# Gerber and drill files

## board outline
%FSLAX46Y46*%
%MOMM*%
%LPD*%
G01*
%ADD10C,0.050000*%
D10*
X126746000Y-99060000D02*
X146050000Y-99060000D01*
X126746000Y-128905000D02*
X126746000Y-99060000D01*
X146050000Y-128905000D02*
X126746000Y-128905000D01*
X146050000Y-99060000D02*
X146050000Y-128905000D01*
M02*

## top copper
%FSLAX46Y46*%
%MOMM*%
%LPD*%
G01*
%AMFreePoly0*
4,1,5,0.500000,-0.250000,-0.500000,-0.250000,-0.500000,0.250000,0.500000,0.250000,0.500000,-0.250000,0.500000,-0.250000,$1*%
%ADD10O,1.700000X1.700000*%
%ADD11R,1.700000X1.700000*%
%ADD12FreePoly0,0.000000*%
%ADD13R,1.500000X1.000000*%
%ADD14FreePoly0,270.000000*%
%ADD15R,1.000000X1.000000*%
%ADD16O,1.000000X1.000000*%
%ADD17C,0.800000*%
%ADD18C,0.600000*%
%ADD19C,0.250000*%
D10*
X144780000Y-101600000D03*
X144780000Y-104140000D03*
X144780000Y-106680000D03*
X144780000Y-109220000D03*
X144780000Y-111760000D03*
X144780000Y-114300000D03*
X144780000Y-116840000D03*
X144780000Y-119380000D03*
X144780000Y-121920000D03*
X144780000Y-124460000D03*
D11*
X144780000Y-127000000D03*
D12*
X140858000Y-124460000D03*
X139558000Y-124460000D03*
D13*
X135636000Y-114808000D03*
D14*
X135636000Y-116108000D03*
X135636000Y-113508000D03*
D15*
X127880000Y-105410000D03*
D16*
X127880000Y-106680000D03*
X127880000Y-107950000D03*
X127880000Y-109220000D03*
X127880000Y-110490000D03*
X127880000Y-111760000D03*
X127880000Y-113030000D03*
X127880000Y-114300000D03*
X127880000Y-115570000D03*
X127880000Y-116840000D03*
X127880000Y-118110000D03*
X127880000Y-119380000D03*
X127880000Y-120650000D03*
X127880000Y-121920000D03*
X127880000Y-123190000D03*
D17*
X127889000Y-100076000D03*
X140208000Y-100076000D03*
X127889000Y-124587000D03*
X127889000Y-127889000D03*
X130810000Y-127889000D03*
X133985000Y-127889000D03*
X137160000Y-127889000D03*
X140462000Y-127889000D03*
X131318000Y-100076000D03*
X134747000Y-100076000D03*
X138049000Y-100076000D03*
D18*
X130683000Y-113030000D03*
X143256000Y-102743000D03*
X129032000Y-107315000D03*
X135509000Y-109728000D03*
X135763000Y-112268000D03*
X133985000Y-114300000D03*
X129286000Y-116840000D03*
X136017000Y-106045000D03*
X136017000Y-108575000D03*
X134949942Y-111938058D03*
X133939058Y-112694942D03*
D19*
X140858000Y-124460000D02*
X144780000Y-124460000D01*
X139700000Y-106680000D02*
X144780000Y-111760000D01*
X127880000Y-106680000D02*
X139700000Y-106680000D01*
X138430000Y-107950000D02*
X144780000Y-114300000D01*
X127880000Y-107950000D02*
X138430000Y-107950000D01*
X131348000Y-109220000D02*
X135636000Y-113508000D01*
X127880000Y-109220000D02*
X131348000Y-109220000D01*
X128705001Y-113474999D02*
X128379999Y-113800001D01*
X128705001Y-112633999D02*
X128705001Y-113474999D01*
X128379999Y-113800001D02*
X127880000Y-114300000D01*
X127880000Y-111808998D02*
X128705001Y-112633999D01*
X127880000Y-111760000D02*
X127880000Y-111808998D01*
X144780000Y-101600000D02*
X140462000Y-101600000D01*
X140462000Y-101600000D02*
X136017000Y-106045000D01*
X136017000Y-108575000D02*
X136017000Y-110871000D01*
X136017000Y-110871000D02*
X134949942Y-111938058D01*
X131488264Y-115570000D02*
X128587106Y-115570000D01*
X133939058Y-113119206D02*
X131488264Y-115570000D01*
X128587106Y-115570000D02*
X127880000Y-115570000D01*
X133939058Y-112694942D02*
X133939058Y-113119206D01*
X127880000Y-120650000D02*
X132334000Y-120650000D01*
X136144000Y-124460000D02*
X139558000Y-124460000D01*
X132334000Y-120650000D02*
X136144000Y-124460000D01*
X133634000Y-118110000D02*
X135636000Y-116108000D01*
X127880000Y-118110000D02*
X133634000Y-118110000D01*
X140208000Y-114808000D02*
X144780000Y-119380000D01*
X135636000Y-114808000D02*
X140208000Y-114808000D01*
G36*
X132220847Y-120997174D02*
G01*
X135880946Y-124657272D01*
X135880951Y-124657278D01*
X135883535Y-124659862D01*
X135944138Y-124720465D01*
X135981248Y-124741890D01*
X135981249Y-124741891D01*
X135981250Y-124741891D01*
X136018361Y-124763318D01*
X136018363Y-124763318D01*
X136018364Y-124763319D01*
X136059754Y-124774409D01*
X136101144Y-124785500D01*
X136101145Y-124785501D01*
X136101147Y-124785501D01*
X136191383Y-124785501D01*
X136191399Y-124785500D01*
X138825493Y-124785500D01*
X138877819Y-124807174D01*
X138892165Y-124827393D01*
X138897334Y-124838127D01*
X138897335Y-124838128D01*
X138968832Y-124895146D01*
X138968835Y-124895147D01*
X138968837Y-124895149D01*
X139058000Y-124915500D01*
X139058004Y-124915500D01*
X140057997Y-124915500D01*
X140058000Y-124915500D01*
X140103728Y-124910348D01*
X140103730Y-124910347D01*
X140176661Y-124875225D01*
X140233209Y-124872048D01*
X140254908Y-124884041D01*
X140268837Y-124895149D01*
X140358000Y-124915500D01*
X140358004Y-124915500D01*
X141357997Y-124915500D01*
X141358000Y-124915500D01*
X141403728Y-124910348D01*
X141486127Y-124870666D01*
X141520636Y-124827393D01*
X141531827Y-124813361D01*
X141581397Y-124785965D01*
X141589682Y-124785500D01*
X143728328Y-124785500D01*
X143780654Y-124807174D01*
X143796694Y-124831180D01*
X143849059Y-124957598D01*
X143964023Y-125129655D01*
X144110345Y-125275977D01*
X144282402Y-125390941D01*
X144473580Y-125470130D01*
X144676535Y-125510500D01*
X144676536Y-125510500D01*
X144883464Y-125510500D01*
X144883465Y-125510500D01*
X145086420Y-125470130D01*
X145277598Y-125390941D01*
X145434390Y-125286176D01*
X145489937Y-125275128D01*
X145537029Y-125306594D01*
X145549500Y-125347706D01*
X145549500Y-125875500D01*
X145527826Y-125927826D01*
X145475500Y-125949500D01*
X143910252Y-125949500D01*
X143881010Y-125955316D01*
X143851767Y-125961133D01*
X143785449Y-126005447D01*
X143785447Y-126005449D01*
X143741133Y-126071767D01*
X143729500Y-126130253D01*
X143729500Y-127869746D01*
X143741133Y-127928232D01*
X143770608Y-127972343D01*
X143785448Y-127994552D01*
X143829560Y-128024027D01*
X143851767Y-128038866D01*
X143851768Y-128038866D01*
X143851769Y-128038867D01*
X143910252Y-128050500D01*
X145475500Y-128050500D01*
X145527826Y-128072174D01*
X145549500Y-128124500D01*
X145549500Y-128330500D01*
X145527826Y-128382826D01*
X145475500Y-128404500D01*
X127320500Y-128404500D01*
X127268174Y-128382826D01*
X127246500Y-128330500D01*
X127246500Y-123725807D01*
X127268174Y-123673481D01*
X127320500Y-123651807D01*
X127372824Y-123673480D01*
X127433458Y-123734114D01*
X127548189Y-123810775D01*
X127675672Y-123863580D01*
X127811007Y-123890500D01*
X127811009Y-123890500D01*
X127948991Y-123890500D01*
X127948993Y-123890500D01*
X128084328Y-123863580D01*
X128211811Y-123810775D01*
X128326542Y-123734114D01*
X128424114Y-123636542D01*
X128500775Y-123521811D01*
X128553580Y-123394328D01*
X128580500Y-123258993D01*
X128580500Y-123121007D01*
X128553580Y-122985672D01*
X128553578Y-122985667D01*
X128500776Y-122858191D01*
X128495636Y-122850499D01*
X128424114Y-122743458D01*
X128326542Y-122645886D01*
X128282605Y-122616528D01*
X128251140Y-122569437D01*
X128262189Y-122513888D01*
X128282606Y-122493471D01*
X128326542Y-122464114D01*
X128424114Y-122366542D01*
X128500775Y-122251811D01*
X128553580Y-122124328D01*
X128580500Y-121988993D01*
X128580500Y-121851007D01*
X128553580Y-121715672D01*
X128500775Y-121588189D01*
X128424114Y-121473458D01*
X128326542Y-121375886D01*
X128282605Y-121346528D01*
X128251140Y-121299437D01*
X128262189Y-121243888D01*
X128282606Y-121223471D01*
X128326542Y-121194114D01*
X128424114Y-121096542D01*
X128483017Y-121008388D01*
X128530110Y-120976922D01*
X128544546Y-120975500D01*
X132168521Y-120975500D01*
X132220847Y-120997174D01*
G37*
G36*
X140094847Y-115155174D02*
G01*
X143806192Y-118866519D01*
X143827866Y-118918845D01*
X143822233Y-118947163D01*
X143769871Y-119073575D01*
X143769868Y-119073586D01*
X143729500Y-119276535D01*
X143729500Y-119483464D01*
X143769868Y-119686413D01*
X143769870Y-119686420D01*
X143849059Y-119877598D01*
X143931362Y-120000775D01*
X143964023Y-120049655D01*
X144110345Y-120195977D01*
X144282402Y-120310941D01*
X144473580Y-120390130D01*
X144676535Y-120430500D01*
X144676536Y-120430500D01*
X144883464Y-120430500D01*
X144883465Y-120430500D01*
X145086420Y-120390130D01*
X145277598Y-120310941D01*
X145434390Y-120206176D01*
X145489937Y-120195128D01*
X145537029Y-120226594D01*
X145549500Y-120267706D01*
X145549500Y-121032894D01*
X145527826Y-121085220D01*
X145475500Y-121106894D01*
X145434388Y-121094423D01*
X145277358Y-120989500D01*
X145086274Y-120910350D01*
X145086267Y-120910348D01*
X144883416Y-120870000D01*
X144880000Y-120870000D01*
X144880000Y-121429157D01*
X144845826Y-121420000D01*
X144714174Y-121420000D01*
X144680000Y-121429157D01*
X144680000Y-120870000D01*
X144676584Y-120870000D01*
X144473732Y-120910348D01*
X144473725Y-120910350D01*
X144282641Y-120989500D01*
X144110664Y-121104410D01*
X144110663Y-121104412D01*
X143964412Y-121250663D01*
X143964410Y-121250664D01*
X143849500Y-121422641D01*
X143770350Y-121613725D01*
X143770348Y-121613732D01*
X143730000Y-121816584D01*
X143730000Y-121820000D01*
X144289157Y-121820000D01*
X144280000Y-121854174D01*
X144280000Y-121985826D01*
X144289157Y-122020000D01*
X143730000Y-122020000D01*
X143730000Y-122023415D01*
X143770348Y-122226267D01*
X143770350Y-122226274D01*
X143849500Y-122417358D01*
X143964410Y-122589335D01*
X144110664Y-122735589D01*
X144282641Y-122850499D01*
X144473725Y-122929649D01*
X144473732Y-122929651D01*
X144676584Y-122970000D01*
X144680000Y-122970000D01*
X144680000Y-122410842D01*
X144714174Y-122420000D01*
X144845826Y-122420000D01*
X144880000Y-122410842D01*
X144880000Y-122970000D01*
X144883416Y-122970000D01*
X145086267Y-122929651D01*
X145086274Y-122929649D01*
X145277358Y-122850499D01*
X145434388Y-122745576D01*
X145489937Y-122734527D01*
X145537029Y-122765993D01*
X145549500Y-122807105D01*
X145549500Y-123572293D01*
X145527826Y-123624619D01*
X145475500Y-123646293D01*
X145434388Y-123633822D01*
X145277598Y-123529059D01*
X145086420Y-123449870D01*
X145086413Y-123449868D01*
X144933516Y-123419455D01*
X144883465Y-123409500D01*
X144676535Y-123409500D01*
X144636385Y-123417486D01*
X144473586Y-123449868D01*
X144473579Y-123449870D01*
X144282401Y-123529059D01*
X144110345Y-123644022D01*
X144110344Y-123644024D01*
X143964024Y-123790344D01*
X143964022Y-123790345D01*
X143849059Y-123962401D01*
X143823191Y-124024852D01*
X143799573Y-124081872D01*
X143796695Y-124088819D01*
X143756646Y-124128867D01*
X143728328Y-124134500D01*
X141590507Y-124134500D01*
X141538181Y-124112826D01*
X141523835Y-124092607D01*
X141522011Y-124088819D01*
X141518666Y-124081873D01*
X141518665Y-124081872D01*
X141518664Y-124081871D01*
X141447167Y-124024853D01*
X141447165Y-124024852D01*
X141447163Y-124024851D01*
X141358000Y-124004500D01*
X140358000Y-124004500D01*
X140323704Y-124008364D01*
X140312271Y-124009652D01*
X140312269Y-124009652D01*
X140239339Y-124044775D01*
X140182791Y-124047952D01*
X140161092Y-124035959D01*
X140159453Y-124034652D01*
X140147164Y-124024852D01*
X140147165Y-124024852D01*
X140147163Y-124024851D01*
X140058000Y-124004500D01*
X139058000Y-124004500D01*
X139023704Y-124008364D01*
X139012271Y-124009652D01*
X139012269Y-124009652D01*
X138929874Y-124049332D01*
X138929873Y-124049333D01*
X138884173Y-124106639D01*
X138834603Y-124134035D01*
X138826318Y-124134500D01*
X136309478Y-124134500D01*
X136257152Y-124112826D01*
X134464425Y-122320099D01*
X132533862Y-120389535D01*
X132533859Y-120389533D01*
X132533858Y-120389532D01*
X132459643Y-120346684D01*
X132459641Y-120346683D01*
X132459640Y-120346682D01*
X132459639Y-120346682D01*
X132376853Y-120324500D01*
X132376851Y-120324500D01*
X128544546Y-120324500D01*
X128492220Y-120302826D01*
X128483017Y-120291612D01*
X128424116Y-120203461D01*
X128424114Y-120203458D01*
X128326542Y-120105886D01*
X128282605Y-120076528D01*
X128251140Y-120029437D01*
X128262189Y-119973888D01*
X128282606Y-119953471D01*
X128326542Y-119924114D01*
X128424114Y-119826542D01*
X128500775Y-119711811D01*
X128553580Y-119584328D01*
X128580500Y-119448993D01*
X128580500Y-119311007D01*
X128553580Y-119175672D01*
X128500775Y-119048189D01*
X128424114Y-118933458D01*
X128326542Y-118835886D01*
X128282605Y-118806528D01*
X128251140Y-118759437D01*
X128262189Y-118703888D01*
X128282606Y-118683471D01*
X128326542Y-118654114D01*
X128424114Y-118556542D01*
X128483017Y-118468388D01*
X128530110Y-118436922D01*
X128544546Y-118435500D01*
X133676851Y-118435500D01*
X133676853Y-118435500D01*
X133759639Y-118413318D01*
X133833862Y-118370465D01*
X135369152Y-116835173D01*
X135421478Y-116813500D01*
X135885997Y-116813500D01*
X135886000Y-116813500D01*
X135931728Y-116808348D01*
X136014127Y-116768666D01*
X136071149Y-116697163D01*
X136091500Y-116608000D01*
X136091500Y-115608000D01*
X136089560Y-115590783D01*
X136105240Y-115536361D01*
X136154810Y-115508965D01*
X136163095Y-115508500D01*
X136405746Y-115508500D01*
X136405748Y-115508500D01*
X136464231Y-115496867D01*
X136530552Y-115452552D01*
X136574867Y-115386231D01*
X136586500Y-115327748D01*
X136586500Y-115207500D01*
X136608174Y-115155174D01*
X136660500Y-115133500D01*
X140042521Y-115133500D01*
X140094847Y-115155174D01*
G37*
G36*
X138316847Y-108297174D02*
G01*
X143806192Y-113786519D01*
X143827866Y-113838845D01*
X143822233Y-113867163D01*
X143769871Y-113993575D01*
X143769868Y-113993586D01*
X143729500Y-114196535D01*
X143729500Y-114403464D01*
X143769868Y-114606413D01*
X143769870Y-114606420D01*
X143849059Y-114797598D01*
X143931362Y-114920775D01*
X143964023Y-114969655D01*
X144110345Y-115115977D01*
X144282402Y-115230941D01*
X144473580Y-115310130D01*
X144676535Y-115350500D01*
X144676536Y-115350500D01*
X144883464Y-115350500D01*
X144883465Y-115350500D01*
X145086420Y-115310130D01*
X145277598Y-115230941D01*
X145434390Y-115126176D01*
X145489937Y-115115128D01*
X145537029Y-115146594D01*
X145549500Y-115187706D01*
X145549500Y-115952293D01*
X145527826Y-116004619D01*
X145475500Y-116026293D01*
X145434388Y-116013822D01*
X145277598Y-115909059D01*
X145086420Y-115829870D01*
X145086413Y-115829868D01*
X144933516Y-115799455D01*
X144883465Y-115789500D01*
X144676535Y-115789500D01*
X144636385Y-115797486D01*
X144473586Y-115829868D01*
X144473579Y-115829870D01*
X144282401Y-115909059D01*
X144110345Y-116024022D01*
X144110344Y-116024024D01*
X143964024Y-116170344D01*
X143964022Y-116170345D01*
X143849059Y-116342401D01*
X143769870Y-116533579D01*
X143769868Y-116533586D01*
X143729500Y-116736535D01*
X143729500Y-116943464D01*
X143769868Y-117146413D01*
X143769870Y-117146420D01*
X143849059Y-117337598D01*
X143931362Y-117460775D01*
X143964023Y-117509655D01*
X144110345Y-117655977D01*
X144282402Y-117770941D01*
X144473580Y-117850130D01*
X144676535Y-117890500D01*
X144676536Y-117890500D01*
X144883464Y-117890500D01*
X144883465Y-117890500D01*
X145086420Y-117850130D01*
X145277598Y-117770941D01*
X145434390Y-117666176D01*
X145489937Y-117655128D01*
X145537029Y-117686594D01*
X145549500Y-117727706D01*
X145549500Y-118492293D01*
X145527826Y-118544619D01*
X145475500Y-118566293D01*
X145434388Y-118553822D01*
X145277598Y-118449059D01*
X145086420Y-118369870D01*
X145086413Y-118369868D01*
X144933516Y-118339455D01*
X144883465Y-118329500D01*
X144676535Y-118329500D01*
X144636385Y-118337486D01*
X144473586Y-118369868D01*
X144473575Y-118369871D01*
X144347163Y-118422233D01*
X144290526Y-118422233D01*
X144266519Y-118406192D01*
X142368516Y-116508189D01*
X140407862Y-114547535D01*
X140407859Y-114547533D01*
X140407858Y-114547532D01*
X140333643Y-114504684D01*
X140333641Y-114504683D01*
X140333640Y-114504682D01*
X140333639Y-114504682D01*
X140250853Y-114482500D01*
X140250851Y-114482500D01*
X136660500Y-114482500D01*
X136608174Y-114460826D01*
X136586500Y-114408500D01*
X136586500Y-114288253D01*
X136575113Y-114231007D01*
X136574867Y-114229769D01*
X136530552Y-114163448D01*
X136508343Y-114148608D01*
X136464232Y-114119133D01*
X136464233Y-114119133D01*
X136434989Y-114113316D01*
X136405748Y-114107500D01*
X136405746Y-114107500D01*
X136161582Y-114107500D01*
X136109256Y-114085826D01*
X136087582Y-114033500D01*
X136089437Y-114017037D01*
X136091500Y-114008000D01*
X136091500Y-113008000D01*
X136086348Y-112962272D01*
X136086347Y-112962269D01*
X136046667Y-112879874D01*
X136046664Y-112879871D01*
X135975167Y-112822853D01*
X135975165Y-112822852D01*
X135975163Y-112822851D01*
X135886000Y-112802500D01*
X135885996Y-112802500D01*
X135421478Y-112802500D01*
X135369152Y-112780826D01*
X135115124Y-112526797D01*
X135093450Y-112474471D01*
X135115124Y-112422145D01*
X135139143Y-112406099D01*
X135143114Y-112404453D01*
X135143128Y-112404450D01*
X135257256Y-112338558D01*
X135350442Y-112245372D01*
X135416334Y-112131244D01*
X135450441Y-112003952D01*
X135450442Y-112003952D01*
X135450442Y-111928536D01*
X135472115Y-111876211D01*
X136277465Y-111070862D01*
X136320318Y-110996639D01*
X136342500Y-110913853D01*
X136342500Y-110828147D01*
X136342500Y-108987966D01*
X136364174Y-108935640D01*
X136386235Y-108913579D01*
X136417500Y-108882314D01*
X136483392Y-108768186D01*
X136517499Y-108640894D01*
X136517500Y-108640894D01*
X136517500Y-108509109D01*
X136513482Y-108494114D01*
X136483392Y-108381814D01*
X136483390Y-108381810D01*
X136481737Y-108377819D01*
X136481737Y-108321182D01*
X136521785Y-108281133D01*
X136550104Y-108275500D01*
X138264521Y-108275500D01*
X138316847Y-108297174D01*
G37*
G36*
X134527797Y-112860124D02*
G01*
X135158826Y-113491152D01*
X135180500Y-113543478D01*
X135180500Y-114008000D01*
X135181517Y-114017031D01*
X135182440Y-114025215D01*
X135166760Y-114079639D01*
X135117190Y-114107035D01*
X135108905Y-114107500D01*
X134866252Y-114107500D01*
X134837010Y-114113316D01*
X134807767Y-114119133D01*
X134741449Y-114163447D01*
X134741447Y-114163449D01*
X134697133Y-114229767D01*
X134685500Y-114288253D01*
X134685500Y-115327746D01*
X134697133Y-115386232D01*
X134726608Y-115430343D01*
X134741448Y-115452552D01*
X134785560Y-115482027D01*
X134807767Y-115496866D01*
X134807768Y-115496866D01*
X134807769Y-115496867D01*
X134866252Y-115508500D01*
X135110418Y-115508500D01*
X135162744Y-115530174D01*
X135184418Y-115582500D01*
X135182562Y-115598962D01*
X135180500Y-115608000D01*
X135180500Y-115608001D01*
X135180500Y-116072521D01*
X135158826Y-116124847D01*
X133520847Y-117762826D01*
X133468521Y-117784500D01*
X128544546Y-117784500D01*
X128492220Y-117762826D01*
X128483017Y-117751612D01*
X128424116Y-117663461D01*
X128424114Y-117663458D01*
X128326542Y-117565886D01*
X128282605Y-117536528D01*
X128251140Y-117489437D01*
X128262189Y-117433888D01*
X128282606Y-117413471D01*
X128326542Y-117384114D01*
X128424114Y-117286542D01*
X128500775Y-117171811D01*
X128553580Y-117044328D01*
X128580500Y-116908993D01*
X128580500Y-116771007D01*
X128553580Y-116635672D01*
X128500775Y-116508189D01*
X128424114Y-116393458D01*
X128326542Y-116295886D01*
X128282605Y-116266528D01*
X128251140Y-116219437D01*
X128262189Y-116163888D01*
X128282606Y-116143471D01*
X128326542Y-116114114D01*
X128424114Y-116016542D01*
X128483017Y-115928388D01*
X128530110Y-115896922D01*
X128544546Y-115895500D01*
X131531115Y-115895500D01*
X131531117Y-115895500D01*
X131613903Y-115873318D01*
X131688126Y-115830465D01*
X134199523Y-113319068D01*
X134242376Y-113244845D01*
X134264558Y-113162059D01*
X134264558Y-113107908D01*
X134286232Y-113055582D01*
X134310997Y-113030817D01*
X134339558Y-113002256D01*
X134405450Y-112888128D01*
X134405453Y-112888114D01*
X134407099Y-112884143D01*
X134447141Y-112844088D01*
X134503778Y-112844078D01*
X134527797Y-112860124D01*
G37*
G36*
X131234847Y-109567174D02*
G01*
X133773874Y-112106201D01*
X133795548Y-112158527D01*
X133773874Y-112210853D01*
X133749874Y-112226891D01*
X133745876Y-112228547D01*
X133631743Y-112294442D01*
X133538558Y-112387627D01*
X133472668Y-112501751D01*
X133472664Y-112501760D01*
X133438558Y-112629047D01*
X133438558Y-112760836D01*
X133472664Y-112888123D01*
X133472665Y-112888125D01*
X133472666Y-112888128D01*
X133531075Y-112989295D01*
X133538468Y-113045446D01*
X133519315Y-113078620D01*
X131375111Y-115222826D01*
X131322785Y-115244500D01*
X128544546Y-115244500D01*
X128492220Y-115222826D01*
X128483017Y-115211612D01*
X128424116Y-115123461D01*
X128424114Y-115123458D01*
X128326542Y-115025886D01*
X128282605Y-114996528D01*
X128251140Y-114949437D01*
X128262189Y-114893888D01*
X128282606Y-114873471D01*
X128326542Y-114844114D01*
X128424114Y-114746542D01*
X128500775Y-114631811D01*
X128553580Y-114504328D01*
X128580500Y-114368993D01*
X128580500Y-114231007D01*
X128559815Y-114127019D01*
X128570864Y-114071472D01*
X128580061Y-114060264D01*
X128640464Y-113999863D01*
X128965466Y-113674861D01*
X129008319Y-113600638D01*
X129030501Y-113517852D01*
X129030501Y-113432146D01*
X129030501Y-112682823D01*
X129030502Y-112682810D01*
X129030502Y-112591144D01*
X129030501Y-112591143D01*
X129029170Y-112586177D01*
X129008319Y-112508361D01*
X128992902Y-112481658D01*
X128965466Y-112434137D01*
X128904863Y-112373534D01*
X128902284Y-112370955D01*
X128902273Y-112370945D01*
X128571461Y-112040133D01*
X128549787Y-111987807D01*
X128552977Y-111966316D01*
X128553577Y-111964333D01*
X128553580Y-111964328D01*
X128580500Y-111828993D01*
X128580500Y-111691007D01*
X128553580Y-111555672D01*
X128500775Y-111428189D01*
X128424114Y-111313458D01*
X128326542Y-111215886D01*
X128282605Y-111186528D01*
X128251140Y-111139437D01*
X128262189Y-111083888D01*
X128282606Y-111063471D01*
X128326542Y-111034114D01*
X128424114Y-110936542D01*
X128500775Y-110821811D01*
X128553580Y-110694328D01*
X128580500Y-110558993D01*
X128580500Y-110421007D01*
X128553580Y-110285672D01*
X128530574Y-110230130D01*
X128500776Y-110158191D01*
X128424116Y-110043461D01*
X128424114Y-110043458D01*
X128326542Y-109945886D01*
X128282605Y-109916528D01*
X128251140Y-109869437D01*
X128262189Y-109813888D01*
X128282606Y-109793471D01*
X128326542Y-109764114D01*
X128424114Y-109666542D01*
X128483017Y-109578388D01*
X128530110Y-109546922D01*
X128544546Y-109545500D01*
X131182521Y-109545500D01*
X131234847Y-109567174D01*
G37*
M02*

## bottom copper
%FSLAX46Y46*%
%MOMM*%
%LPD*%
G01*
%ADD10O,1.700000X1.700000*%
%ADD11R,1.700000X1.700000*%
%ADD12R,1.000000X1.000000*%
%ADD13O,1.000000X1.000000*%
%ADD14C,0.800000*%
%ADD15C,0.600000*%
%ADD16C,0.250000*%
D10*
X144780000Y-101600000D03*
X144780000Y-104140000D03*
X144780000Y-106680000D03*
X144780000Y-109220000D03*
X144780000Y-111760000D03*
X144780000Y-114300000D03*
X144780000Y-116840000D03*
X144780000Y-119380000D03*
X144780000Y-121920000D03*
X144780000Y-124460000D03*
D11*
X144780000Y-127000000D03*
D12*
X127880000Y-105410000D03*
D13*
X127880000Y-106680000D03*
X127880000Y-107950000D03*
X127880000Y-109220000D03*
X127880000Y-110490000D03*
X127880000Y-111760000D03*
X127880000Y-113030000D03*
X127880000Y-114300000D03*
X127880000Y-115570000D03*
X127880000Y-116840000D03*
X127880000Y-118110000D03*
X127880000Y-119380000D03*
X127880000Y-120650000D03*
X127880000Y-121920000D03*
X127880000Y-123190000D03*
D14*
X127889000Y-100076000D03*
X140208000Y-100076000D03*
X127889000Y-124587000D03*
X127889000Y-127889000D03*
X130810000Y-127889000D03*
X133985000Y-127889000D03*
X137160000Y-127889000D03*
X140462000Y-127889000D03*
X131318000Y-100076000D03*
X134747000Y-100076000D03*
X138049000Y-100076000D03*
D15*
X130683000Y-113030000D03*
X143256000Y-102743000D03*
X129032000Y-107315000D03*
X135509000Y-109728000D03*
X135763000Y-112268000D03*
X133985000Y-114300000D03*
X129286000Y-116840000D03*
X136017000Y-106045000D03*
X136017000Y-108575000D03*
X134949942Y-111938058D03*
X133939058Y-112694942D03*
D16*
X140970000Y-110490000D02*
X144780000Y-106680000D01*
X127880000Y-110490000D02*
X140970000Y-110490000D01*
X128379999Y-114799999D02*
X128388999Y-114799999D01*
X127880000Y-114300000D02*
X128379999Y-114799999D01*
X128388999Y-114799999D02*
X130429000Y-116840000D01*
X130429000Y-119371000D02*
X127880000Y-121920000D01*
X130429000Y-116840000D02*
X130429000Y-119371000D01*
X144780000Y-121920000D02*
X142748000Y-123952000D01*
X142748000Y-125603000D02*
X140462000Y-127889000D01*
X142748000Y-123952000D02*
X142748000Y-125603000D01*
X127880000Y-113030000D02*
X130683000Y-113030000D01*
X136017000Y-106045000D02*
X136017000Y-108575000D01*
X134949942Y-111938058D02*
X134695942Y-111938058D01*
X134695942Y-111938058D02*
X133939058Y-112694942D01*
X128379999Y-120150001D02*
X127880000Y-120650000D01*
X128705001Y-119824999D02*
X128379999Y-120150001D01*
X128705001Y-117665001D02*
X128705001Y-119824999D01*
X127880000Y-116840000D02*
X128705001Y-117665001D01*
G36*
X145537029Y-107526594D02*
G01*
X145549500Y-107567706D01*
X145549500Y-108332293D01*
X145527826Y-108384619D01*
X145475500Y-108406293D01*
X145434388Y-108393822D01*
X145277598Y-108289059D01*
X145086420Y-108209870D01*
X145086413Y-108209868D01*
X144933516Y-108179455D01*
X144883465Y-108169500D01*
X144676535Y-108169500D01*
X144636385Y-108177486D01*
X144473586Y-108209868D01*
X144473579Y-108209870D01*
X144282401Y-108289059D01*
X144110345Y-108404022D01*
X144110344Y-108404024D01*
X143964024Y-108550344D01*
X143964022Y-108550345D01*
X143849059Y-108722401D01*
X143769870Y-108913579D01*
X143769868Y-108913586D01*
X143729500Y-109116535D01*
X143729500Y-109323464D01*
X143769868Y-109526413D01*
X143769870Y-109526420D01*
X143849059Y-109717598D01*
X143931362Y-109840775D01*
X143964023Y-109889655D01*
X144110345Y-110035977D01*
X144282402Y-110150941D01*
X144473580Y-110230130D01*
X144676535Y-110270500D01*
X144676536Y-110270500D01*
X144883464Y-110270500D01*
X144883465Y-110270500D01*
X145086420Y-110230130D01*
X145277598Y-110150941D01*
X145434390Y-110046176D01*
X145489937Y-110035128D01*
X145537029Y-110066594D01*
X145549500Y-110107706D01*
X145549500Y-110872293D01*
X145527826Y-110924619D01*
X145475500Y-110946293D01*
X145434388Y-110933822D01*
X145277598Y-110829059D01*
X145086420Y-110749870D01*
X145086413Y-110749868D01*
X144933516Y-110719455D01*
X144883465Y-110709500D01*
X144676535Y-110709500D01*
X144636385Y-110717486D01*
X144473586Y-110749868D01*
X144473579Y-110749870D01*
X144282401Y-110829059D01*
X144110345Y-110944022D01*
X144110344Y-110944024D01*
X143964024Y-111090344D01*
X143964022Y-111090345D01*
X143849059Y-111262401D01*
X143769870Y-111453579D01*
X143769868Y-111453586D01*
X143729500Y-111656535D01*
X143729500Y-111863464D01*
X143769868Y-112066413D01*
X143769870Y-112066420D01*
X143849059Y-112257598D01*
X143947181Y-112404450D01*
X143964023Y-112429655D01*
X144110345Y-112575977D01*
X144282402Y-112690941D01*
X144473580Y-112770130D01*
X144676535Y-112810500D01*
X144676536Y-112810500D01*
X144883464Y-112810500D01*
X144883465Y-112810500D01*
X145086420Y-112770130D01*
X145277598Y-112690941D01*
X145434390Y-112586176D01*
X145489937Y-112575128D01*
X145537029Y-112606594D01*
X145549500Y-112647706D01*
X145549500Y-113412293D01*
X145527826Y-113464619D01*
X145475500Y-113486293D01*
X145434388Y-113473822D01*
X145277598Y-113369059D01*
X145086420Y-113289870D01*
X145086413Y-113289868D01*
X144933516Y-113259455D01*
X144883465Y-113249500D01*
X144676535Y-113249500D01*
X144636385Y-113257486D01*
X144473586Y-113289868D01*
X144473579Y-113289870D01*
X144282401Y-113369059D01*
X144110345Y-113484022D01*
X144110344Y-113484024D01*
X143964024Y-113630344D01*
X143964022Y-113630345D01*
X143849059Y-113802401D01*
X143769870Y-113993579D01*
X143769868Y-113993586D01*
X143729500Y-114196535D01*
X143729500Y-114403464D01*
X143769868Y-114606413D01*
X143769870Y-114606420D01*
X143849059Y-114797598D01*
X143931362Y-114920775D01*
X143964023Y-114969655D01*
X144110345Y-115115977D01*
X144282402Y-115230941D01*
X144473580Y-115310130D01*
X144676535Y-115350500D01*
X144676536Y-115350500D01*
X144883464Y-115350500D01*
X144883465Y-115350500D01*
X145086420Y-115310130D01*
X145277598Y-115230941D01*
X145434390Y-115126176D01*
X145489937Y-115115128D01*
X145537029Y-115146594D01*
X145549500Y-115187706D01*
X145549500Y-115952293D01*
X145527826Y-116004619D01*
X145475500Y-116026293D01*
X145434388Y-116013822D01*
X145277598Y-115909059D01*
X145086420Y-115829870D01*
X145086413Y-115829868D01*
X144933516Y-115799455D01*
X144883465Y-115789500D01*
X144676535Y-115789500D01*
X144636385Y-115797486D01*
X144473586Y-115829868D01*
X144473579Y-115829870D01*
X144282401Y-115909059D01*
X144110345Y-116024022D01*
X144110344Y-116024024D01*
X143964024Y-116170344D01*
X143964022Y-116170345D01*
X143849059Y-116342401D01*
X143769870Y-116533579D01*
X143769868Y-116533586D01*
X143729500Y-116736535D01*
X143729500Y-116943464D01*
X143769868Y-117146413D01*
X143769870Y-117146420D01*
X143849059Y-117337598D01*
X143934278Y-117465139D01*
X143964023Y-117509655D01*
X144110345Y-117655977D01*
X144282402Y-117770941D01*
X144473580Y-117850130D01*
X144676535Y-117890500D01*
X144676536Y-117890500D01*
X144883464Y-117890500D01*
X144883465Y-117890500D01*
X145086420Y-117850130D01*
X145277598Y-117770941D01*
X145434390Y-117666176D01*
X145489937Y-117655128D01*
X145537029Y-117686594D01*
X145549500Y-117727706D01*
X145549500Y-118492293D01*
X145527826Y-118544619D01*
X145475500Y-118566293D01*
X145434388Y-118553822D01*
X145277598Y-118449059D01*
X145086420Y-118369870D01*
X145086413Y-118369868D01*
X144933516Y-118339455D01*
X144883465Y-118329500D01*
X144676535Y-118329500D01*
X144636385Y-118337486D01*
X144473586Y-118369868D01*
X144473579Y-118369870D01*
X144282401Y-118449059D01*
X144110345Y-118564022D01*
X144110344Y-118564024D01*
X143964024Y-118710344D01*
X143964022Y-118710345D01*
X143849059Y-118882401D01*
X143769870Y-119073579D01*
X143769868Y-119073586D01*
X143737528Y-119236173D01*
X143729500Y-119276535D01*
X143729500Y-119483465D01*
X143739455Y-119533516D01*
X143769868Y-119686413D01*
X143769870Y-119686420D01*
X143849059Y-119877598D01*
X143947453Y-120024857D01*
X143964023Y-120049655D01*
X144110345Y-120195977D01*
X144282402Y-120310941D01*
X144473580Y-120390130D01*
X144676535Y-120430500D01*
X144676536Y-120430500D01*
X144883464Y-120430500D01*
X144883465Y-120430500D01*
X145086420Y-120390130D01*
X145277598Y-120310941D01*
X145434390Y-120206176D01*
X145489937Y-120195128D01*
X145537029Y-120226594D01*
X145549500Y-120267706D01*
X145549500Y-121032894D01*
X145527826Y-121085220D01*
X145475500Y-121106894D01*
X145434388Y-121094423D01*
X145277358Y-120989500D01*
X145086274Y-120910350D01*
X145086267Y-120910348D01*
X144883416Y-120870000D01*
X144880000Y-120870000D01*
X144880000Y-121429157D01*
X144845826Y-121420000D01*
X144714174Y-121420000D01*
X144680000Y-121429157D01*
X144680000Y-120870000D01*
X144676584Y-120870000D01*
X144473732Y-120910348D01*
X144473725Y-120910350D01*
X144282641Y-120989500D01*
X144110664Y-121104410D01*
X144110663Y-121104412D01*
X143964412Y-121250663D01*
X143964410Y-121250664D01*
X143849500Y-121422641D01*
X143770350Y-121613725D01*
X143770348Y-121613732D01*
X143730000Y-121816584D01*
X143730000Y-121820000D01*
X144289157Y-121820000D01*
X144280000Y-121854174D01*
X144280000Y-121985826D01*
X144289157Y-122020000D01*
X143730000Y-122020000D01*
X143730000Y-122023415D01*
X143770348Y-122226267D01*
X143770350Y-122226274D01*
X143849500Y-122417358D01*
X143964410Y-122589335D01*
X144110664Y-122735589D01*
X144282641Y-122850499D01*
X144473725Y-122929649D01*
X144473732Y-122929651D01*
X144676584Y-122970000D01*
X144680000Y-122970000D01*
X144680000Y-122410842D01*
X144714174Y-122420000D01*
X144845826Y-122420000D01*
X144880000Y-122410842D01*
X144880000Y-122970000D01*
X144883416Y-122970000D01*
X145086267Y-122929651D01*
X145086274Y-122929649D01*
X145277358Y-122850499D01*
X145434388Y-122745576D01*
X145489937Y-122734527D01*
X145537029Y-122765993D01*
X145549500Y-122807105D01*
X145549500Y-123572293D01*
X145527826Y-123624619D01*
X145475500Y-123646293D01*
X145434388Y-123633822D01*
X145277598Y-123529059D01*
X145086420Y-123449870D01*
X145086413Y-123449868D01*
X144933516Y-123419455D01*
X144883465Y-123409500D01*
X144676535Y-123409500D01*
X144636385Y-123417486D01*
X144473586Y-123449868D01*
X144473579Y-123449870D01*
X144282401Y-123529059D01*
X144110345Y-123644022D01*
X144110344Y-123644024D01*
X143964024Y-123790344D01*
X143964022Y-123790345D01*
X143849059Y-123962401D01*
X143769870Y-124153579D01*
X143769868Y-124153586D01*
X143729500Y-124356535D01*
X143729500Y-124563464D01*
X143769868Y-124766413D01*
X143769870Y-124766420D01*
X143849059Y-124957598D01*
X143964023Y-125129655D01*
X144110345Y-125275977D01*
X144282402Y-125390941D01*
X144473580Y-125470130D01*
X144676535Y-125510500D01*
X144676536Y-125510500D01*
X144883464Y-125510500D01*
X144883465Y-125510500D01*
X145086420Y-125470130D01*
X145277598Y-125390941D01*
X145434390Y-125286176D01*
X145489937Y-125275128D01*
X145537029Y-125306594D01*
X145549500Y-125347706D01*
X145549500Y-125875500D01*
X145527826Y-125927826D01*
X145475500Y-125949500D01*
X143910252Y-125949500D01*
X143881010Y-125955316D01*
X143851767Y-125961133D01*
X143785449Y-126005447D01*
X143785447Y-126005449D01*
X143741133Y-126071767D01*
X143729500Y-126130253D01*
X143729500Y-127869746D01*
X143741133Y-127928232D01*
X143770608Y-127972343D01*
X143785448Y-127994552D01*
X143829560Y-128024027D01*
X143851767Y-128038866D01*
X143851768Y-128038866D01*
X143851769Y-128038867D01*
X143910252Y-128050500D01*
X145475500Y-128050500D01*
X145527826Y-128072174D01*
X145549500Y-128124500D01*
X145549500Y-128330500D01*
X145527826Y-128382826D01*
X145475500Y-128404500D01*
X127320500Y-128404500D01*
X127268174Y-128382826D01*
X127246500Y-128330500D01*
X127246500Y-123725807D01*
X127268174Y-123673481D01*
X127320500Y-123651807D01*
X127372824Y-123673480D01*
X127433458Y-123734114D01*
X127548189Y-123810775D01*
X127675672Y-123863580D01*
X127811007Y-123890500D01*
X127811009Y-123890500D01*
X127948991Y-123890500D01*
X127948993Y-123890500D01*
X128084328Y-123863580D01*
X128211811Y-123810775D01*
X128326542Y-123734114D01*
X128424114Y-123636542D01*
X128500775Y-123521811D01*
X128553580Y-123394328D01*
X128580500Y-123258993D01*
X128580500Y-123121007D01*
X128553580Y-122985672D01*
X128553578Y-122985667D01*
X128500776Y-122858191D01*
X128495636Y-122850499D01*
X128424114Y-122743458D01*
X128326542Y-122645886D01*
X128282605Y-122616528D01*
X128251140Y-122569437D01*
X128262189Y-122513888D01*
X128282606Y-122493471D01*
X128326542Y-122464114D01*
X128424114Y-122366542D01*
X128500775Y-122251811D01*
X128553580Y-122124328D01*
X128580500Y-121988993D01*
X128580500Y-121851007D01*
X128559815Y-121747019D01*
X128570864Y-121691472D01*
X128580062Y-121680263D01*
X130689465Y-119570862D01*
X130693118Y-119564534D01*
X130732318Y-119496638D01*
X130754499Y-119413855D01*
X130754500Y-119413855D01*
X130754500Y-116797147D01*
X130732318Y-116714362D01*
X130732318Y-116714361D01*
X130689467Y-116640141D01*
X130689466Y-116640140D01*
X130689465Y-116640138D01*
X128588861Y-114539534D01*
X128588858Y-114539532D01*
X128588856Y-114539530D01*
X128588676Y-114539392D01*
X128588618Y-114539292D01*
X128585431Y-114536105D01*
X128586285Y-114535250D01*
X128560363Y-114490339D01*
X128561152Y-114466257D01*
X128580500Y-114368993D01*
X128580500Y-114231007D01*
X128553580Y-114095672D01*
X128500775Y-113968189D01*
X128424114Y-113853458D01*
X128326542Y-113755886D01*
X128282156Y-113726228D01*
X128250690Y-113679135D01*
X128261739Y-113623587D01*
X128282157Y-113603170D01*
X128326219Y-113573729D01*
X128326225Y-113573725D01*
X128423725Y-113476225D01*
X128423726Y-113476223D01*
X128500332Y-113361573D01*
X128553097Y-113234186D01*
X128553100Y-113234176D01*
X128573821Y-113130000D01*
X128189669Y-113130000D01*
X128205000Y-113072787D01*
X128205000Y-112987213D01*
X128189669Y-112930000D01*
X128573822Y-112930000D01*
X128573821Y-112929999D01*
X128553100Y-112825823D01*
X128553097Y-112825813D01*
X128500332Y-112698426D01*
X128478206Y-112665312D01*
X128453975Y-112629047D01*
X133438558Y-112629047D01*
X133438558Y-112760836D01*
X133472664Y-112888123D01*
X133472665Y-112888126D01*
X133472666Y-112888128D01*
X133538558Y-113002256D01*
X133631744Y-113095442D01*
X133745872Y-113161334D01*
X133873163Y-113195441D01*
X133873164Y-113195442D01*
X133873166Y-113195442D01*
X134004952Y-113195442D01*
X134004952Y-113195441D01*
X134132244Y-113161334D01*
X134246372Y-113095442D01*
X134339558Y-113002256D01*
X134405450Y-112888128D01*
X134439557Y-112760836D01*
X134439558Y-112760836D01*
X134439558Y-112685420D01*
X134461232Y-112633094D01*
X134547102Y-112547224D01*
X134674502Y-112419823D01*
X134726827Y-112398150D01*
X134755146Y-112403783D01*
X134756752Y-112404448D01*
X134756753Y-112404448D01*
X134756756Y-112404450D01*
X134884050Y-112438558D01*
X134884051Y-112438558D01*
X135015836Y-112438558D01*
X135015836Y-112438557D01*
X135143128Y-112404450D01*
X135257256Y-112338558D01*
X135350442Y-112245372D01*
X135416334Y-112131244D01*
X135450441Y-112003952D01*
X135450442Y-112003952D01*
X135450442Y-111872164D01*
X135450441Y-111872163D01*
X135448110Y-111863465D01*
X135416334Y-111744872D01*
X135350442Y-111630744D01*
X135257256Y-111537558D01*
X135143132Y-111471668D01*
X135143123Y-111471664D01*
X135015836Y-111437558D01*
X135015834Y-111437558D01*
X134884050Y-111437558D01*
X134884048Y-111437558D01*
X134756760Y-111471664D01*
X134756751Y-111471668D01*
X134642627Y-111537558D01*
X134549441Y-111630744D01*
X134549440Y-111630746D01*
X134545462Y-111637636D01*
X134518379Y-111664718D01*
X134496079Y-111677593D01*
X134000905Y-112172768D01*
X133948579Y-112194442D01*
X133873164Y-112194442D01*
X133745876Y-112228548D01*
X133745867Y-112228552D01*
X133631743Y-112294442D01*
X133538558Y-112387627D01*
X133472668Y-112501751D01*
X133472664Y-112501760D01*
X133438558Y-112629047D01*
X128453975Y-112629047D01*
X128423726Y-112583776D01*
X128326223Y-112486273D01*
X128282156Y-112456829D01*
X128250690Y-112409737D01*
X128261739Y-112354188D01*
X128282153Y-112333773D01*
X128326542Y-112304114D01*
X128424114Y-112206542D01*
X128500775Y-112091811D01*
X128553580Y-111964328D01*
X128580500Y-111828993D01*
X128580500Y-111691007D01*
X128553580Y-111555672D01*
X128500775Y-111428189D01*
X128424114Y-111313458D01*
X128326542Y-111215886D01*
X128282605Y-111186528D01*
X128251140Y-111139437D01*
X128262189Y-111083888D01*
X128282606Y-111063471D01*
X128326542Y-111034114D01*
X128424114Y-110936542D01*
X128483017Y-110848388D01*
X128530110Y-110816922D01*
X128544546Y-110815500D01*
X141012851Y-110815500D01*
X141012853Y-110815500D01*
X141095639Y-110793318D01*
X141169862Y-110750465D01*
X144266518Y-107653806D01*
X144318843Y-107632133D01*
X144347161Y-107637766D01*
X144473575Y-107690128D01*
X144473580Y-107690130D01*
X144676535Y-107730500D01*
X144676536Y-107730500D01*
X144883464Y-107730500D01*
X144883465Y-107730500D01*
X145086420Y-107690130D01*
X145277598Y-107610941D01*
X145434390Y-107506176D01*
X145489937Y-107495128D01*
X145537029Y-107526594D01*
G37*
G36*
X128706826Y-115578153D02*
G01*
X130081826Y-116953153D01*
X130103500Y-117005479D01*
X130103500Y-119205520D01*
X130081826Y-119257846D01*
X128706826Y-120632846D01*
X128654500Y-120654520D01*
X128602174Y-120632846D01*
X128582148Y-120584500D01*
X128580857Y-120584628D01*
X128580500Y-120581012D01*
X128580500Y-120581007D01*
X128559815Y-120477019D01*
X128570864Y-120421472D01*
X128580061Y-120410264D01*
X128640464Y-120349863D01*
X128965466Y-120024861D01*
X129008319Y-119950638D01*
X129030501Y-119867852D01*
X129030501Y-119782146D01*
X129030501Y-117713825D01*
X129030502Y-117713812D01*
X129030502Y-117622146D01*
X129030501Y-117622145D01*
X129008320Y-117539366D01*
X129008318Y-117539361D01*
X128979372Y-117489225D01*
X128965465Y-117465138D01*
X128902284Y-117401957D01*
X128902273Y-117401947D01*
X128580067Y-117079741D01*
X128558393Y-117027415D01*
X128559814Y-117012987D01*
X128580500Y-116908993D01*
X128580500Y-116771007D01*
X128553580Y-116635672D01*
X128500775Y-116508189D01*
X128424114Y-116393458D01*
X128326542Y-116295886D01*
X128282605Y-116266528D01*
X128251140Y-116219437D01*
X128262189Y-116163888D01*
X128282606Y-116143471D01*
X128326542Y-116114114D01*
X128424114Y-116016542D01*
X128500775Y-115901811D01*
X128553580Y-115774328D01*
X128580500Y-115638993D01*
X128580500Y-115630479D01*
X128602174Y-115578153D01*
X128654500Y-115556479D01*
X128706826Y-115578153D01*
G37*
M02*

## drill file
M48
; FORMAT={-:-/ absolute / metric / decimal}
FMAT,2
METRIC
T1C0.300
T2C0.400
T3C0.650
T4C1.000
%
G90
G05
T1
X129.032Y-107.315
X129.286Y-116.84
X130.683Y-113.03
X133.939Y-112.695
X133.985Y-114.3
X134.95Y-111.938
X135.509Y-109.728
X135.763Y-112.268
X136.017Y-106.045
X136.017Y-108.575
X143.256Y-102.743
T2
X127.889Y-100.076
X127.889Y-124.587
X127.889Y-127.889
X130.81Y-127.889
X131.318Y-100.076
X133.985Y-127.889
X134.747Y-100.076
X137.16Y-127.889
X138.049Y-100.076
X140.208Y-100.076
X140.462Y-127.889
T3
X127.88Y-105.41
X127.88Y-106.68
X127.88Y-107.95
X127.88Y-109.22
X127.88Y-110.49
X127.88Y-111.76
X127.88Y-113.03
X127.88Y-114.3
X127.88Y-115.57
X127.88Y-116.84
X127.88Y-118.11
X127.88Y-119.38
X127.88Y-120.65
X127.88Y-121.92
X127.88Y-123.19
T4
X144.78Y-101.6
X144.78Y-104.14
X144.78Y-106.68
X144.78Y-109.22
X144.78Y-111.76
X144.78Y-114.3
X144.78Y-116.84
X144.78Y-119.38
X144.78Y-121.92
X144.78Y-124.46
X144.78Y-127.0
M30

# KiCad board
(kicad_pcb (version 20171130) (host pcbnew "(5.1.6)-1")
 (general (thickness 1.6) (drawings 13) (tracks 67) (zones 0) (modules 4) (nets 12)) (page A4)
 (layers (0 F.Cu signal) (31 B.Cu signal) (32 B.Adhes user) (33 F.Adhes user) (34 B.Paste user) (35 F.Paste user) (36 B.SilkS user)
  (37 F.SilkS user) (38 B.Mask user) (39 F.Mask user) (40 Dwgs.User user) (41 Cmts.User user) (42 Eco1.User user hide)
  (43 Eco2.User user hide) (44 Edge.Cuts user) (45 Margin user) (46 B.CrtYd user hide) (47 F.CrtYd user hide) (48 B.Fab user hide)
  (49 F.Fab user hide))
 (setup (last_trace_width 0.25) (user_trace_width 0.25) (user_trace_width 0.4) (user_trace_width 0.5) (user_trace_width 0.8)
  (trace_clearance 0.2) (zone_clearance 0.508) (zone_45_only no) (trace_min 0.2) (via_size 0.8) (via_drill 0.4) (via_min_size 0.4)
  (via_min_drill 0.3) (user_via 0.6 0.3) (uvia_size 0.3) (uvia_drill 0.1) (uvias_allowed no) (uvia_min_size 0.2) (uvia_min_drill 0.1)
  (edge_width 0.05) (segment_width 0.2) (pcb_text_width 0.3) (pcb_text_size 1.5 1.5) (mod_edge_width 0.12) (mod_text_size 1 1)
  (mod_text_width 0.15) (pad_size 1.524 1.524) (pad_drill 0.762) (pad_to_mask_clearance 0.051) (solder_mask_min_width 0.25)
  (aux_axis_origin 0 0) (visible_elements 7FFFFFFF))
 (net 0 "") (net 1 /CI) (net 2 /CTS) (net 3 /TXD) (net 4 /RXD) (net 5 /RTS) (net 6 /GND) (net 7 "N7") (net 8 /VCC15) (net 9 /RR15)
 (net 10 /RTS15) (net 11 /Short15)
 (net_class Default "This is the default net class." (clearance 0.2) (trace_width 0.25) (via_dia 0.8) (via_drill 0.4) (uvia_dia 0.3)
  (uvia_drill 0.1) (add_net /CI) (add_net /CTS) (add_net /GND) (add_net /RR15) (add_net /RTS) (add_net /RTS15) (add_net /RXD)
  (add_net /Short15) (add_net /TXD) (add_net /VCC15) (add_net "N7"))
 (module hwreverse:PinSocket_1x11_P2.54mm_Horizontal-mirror (layer F.Cu) (at 156.14004 107.06862)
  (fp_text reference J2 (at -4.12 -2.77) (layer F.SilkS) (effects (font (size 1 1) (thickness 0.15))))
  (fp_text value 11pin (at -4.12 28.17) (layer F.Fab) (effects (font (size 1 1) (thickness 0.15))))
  (pad 11 thru_hole oval (at -11.36004 -5.46862 180) (size 1.7 1.7) (drill 1) (layers *.Cu *.Mask) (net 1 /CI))
  (pad 10 thru_hole oval (at -11.36004 -2.92862 180) (size 1.7 1.7) (drill 1) (layers *.Cu *.Mask))
  (pad 9 thru_hole oval (at -11.36004 -0.38862 180) (size 1.7 1.7) (drill 1) (layers *.Cu *.Mask) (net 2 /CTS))
  (pad 8 thru_hole oval (at -11.36004 2.15138 180) (size 1.7 1.7) (drill 1) (layers *.Cu *.Mask))
  (pad 7 thru_hole oval (at -11.36004 4.69138 180) (size 1.7 1.7) (drill 1) (layers *.Cu *.Mask) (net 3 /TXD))
  (pad 6 thru_hole oval (at -11.36004 7.23138 180) (size 1.7 1.7) (drill 1) (layers *.Cu *.Mask) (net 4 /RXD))
  (pad 5 thru_hole oval (at -11.36004 9.77138 180) (size 1.7 1.7) (drill 1) (layers *.Cu *.Mask))
  (pad 4 thru_hole oval (at -11.36004 12.31138 180) (size 1.7 1.7) (drill 1) (layers *.Cu *.Mask) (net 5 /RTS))
  (pad 3 thru_hole oval (at -11.36004 14.85138 180) (size 1.7 1.7) (drill 1) (layers *.Cu *.Mask) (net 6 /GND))
  (pad 2 thru_hole oval (at -11.36004 17.39138 180) (size 1.7 1.7) (drill 1) (layers *.Cu *.Mask) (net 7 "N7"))
  (pad 1 thru_hole rect (at -11.36004 19.93138 180) (size 1.7 1.7) (drill 1) (layers *.Cu *.Mask)))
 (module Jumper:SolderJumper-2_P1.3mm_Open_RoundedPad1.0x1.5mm (layer F.Cu) (at 140.208 124.46)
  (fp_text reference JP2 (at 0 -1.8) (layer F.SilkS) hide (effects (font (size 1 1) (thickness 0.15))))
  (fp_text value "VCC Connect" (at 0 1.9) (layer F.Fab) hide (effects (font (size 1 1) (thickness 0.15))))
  (pad 2 smd custom (at 0.65 0) (size 1 0.5) (layers F.Cu F.Mask) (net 7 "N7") (zone_connect 2) (options (clearance outline) (anchor rect))
   (primitives))
  (pad 1 smd custom (at -0.65 0) (size 1 0.5) (layers F.Cu F.Mask) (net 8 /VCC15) (zone_connect 2)
   (options (clearance outline) (anchor rect)) (primitives)))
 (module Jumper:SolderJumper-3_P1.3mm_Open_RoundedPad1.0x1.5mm (layer F.Cu) (at 135.636 114.808 270)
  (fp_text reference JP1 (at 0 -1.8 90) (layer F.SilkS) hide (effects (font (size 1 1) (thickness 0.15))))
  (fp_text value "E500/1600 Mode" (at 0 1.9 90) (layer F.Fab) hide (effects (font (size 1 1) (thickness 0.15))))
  (pad 2 smd rect (at 0 0 270) (size 1 1.5) (layers F.Cu F.Mask) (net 5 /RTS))
  (pad 3 smd custom (at 1.3 0 270) (size 1 0.5) (layers F.Cu F.Mask) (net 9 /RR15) (zone_connect 2)
   (options (clearance outline) (anchor rect)) (primitives))
  (pad 1 smd custom (at -1.3 0 270) (size 1 0.5) (layers F.Cu F.Mask) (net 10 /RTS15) (zone_connect 2)
   (options (clearance outline) (anchor rect)) (primitives)))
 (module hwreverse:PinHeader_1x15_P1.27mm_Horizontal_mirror (layer F.Cu) (at 119.38 105.41)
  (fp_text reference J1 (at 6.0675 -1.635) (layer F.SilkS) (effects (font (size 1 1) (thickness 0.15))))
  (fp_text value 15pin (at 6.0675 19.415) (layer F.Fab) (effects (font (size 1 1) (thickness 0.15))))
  (pad 1 thru_hole rect (at 8.5 0) (size 1 1) (drill 0.65) (layers *.Cu *.Mask))
  (pad 2 thru_hole oval (at 8.5 1.27) (size 1 1) (drill 0.65) (layers *.Cu *.Mask) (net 3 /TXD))
  (pad 3 thru_hole oval (at 8.5 2.54) (size 1 1) (drill 0.65) (layers *.Cu *.Mask) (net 4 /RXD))
  (pad 4 thru_hole oval (at 8.5 3.81) (size 1 1) (drill 0.65) (layers *.Cu *.Mask) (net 10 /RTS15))
  (pad 5 thru_hole oval (at 8.5 5.08) (size 1 1) (drill 0.65) (layers *.Cu *.Mask) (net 2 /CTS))
  (pad 6 thru_hole oval (at 8.5 6.35) (size 1 1) (drill 0.65) (layers *.Cu *.Mask) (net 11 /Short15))
  (pad 7 thru_hole oval (at 8.5 7.62) (size 1 1) (drill 0.65) (layers *.Cu *.Mask) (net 6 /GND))
  (pad 8 thru_hole oval (at 8.5 8.89) (size 1 1) (drill 0.65) (layers *.Cu *.Mask) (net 11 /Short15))
  (pad 9 thru_hole oval (at 8.5 10.16) (size 1 1) (drill 0.65) (layers *.Cu *.Mask) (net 1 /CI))
  (pad 10 thru_hole oval (at 8.5 11.43) (size 1 1) (drill 0.65) (layers *.Cu *.Mask) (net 8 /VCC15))
  (pad 11 thru_hole oval (at 8.5 12.7) (size 1 1) (drill 0.65) (layers *.Cu *.Mask) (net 9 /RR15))
  (pad 12 thru_hole oval (at 8.5 13.97) (size 1 1) (drill 0.65) (layers *.Cu *.Mask))
  (pad 13 thru_hole oval (at 8.5 15.24) (size 1 1) (drill 0.65) (layers *.Cu *.Mask) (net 8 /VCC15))
  (pad 14 thru_hole oval (at 8.5 16.51) (size 1 1) (drill 0.65) (layers *.Cu *.Mask) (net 11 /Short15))
  (pad 15 thru_hole oval (at 8.5 17.78) (size 1 1) (drill 0.65) (layers *.Cu *.Mask)))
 (gr_line (start 126.746 99.06) (end 146.05 99.06) (layer Edge.Cuts) (width 0.05))
 (gr_line (start 126.746 128.905) (end 126.746 99.06) (layer Edge.Cuts) (width 0.05))
 (gr_line (start 146.05 128.905) (end 126.746 128.905) (layer Edge.Cuts) (width 0.05))
 (gr_line (start 146.05 99.06) (end 146.05 128.905) (layer Edge.Cuts) (width 0.05))
 (segment (start 140.858 124.46) (end 144.78 124.46) (width 0.25) (layer F.Cu) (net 7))
 (segment (start 139.7 106.68) (end 144.78 111.76) (width 0.25) (layer F.Cu) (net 3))
 (segment (start 127.88 106.68) (end 139.7 106.68) (width 0.25) (layer F.Cu) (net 3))
 (segment (start 138.43 107.95) (end 144.78 114.3) (width 0.25) (layer F.Cu) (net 4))
 (segment (start 127.88 107.95) (end 138.43 107.95) (width 0.25) (layer F.Cu) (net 4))
 (segment (start 131.348 109.22) (end 135.636 113.508) (width 0.25) (layer F.Cu) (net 10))
 (segment (start 127.88 109.22) (end 131.348 109.22) (width 0.25) (layer F.Cu) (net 10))
 (segment (start 140.97 110.49) (end 144.78 106.68) (width 0.25) (layer B.Cu) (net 2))
 (segment (start 127.88 110.49) (end 140.97 110.49) (width 0.25) (layer B.Cu) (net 2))
 (segment (start 128.705001 113.474999) (end 128.379999 113.800001) (width 0.25) (layer F.Cu) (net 11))
 (segment (start 128.705001 112.633999) (end 128.705001 113.474999) (width 0.25) (layer F.Cu) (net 11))
 (segment (start 128.379999 113.800001) (end 127.88 114.3) (width 0.25) (layer F.Cu) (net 11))
 (segment (start 127.88 111.808998) (end 128.705001 112.633999) (width 0.25) (layer F.Cu) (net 11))
 (segment (start 127.88 111.76) (end 127.88 111.808998) (width 0.25) (layer F.Cu) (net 11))
 (segment (start 128.379999 114.799999) (end 128.388999 114.799999) (width 0.25) (layer B.Cu) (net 11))
 (segment (start 127.88 114.3) (end 128.379999 114.799999) (width 0.25) (layer B.Cu) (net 11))
 (segment (start 128.388999 114.799999) (end 130.429 116.84) (width 0.25) (layer B.Cu) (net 11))
 (segment (start 130.429 119.371) (end 127.88 121.92) (width 0.25) (layer B.Cu) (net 11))
 (segment (start 130.429 116.84) (end 130.429 119.371) (width 0.25) (layer B.Cu) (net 11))
 (via (at 127.889 100.076) (size 0.8) (drill 0.4) (layers F.Cu B.Cu) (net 6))
 (via (at 140.208 100.076) (size 0.8) (drill 0.4) (layers F.Cu B.Cu) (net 6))
 (via (at 127.889 124.587) (size 0.8) (drill 0.4) (layers F.Cu B.Cu) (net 6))
 (via (at 127.889 127.889) (size 0.8) (drill 0.4) (layers F.Cu B.Cu) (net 6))
 (via (at 130.81 127.889) (size 0.8) (drill 0.4) (layers F.Cu B.Cu) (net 6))
 (via (at 133.985 127.889) (size 0.8) (drill 0.4) (layers F.Cu B.Cu) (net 6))
 (via (at 137.16 127.889) (size 0.8) (drill 0.4) (layers F.Cu B.Cu) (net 6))
 (via (at 140.462 127.889) (size 0.8) (drill 0.4) (layers F.Cu B.Cu) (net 6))
 (via (at 131.318 100.076) (size 0.8) (drill 0.4) (layers F.Cu B.Cu) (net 6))
 (via (at 134.747 100.076) (size 0.8) (drill 0.4) (layers F.Cu B.Cu) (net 6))
 (via (at 138.049 100.076) (size 0.8) (drill 0.4) (layers F.Cu B.Cu) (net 6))
 (segment (start 144.78 121.92) (end 142.748 123.952) (width 0.25) (layer B.Cu) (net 6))
 (segment (start 142.748 125.603) (end 140.462 127.889) (width 0.25) (layer B.Cu) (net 6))
 (segment (start 142.748 123.952) (end 142.748 125.603) (width 0.25) (layer B.Cu) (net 6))
 (via (at 130.683 113.03) (size 0.6) (drill 0.3) (layers F.Cu B.Cu) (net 6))
 (segment (start 127.88 113.03) (end 130.683 113.03) (width 0.25) (layer B.Cu) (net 6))
 (via (at 143.256 102.743) (size 0.6) (drill 0.3) (layers F.Cu B.Cu) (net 6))
 (via (at 129.032 107.315) (size 0.6) (drill 0.3) (layers F.Cu B.Cu) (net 6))
 (via (at 135.509 109.728) (size 0.6) (drill 0.3) (layers F.Cu B.Cu) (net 6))
 (via (at 135.763 112.268) (size 0.6) (drill 0.3) (layers F.Cu B.Cu) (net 6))
 (via (at 133.985 114.3) (size 0.6) (drill 0.3) (layers F.Cu B.Cu) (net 6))
 (via (at 129.286 116.84) (size 0.6) (drill 0.3) (layers F.Cu B.Cu) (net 6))
 (via (at 136.017 106.045) (size 0.6) (drill 0.3) (layers F.Cu B.Cu) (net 1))
 (segment (start 144.78 101.6) (end 140.462 101.6) (width 0.25) (layer F.Cu) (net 1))
 (segment (start 140.462 101.6) (end 136.017 106.045) (width 0.25) (layer F.Cu) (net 1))
 (via (at 136.017 108.575) (size 0.6) (drill 0.3) (layers F.Cu B.Cu) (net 1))
 (segment (start 136.017 106.045) (end 136.017 108.575) (width 0.25) (layer B.Cu) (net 1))
 (segment (start 136.017 108.575) (end 136.017 110.871) (width 0.25) (layer F.Cu) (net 1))
 (via (at 134.949942 111.938058) (size 0.6) (drill 0.3) (layers F.Cu B.Cu) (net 1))
 (segment (start 136.017 110.871) (end 134.949942 111.938058) (width 0.25) (layer F.Cu) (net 1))
 (via (at 133.939058 112.694942) (size 0.6) (drill 0.3) (layers F.Cu B.Cu) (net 1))
 (segment (start 134.949942 111.938058) (end 134.695942 111.938058) (width 0.25) (layer B.Cu) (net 1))
 (segment (start 134.695942 111.938058) (end 133.939058 112.694942) (width 0.25) (layer B.Cu) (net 1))
 (segment (start 131.488264 115.57) (end 128.587106 115.57) (width 0.25) (layer F.Cu) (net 1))
 (segment (start 133.939058 113.119206) (end 131.488264 115.57) (width 0.25) (layer F.Cu) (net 1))
 (segment (start 128.587106 115.57) (end 127.88 115.57) (width 0.25) (layer F.Cu) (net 1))
 (segment (start 133.939058 112.694942) (end 133.939058 113.119206) (width 0.25) (layer F.Cu) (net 1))
 (segment (start 127.88 120.65) (end 132.334 120.65) (width 0.25) (layer F.Cu) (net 8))
 (segment (start 136.144 124.46) (end 139.558 124.46) (width 0.25) (layer F.Cu) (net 8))
 (segment (start 132.334 120.65) (end 136.144 124.46) (width 0.25) (layer F.Cu) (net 8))
 (segment (start 128.379999 120.150001) (end 127.88 120.65) (width 0.25) (layer B.Cu) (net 8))
 (segment (start 128.705001 119.824999) (end 128.379999 120.150001) (width 0.25) (layer B.Cu) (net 8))
 (segment (start 128.705001 117.665001) (end 128.705001 119.824999) (width 0.25) (layer B.Cu) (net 8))
 (segment (start 127.88 116.84) (end 128.705001 117.665001) (width 0.25) (layer B.Cu) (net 8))
 (segment (start 133.634 118.11) (end 135.636 116.108) (width 0.25) (layer F.Cu) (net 9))
 (segment (start 127.88 118.11) (end 133.634 118.11) (width 0.25) (layer F.Cu) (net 9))
 (segment (start 140.208 114.808) (end 144.78 119.38) (width 0.25) (layer F.Cu) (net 5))
 (segment (start 135.636 114.808) (end 140.208 114.808) (width 0.25) (layer F.Cu) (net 5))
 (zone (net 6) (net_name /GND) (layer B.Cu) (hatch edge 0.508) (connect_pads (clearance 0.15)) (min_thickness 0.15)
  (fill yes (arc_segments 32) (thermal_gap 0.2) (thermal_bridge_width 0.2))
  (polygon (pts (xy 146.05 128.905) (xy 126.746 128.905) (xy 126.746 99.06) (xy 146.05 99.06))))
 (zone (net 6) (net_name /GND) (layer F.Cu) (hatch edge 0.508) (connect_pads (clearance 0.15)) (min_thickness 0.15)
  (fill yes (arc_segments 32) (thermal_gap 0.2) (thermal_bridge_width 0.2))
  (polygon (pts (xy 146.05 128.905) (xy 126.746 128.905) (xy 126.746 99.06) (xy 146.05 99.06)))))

